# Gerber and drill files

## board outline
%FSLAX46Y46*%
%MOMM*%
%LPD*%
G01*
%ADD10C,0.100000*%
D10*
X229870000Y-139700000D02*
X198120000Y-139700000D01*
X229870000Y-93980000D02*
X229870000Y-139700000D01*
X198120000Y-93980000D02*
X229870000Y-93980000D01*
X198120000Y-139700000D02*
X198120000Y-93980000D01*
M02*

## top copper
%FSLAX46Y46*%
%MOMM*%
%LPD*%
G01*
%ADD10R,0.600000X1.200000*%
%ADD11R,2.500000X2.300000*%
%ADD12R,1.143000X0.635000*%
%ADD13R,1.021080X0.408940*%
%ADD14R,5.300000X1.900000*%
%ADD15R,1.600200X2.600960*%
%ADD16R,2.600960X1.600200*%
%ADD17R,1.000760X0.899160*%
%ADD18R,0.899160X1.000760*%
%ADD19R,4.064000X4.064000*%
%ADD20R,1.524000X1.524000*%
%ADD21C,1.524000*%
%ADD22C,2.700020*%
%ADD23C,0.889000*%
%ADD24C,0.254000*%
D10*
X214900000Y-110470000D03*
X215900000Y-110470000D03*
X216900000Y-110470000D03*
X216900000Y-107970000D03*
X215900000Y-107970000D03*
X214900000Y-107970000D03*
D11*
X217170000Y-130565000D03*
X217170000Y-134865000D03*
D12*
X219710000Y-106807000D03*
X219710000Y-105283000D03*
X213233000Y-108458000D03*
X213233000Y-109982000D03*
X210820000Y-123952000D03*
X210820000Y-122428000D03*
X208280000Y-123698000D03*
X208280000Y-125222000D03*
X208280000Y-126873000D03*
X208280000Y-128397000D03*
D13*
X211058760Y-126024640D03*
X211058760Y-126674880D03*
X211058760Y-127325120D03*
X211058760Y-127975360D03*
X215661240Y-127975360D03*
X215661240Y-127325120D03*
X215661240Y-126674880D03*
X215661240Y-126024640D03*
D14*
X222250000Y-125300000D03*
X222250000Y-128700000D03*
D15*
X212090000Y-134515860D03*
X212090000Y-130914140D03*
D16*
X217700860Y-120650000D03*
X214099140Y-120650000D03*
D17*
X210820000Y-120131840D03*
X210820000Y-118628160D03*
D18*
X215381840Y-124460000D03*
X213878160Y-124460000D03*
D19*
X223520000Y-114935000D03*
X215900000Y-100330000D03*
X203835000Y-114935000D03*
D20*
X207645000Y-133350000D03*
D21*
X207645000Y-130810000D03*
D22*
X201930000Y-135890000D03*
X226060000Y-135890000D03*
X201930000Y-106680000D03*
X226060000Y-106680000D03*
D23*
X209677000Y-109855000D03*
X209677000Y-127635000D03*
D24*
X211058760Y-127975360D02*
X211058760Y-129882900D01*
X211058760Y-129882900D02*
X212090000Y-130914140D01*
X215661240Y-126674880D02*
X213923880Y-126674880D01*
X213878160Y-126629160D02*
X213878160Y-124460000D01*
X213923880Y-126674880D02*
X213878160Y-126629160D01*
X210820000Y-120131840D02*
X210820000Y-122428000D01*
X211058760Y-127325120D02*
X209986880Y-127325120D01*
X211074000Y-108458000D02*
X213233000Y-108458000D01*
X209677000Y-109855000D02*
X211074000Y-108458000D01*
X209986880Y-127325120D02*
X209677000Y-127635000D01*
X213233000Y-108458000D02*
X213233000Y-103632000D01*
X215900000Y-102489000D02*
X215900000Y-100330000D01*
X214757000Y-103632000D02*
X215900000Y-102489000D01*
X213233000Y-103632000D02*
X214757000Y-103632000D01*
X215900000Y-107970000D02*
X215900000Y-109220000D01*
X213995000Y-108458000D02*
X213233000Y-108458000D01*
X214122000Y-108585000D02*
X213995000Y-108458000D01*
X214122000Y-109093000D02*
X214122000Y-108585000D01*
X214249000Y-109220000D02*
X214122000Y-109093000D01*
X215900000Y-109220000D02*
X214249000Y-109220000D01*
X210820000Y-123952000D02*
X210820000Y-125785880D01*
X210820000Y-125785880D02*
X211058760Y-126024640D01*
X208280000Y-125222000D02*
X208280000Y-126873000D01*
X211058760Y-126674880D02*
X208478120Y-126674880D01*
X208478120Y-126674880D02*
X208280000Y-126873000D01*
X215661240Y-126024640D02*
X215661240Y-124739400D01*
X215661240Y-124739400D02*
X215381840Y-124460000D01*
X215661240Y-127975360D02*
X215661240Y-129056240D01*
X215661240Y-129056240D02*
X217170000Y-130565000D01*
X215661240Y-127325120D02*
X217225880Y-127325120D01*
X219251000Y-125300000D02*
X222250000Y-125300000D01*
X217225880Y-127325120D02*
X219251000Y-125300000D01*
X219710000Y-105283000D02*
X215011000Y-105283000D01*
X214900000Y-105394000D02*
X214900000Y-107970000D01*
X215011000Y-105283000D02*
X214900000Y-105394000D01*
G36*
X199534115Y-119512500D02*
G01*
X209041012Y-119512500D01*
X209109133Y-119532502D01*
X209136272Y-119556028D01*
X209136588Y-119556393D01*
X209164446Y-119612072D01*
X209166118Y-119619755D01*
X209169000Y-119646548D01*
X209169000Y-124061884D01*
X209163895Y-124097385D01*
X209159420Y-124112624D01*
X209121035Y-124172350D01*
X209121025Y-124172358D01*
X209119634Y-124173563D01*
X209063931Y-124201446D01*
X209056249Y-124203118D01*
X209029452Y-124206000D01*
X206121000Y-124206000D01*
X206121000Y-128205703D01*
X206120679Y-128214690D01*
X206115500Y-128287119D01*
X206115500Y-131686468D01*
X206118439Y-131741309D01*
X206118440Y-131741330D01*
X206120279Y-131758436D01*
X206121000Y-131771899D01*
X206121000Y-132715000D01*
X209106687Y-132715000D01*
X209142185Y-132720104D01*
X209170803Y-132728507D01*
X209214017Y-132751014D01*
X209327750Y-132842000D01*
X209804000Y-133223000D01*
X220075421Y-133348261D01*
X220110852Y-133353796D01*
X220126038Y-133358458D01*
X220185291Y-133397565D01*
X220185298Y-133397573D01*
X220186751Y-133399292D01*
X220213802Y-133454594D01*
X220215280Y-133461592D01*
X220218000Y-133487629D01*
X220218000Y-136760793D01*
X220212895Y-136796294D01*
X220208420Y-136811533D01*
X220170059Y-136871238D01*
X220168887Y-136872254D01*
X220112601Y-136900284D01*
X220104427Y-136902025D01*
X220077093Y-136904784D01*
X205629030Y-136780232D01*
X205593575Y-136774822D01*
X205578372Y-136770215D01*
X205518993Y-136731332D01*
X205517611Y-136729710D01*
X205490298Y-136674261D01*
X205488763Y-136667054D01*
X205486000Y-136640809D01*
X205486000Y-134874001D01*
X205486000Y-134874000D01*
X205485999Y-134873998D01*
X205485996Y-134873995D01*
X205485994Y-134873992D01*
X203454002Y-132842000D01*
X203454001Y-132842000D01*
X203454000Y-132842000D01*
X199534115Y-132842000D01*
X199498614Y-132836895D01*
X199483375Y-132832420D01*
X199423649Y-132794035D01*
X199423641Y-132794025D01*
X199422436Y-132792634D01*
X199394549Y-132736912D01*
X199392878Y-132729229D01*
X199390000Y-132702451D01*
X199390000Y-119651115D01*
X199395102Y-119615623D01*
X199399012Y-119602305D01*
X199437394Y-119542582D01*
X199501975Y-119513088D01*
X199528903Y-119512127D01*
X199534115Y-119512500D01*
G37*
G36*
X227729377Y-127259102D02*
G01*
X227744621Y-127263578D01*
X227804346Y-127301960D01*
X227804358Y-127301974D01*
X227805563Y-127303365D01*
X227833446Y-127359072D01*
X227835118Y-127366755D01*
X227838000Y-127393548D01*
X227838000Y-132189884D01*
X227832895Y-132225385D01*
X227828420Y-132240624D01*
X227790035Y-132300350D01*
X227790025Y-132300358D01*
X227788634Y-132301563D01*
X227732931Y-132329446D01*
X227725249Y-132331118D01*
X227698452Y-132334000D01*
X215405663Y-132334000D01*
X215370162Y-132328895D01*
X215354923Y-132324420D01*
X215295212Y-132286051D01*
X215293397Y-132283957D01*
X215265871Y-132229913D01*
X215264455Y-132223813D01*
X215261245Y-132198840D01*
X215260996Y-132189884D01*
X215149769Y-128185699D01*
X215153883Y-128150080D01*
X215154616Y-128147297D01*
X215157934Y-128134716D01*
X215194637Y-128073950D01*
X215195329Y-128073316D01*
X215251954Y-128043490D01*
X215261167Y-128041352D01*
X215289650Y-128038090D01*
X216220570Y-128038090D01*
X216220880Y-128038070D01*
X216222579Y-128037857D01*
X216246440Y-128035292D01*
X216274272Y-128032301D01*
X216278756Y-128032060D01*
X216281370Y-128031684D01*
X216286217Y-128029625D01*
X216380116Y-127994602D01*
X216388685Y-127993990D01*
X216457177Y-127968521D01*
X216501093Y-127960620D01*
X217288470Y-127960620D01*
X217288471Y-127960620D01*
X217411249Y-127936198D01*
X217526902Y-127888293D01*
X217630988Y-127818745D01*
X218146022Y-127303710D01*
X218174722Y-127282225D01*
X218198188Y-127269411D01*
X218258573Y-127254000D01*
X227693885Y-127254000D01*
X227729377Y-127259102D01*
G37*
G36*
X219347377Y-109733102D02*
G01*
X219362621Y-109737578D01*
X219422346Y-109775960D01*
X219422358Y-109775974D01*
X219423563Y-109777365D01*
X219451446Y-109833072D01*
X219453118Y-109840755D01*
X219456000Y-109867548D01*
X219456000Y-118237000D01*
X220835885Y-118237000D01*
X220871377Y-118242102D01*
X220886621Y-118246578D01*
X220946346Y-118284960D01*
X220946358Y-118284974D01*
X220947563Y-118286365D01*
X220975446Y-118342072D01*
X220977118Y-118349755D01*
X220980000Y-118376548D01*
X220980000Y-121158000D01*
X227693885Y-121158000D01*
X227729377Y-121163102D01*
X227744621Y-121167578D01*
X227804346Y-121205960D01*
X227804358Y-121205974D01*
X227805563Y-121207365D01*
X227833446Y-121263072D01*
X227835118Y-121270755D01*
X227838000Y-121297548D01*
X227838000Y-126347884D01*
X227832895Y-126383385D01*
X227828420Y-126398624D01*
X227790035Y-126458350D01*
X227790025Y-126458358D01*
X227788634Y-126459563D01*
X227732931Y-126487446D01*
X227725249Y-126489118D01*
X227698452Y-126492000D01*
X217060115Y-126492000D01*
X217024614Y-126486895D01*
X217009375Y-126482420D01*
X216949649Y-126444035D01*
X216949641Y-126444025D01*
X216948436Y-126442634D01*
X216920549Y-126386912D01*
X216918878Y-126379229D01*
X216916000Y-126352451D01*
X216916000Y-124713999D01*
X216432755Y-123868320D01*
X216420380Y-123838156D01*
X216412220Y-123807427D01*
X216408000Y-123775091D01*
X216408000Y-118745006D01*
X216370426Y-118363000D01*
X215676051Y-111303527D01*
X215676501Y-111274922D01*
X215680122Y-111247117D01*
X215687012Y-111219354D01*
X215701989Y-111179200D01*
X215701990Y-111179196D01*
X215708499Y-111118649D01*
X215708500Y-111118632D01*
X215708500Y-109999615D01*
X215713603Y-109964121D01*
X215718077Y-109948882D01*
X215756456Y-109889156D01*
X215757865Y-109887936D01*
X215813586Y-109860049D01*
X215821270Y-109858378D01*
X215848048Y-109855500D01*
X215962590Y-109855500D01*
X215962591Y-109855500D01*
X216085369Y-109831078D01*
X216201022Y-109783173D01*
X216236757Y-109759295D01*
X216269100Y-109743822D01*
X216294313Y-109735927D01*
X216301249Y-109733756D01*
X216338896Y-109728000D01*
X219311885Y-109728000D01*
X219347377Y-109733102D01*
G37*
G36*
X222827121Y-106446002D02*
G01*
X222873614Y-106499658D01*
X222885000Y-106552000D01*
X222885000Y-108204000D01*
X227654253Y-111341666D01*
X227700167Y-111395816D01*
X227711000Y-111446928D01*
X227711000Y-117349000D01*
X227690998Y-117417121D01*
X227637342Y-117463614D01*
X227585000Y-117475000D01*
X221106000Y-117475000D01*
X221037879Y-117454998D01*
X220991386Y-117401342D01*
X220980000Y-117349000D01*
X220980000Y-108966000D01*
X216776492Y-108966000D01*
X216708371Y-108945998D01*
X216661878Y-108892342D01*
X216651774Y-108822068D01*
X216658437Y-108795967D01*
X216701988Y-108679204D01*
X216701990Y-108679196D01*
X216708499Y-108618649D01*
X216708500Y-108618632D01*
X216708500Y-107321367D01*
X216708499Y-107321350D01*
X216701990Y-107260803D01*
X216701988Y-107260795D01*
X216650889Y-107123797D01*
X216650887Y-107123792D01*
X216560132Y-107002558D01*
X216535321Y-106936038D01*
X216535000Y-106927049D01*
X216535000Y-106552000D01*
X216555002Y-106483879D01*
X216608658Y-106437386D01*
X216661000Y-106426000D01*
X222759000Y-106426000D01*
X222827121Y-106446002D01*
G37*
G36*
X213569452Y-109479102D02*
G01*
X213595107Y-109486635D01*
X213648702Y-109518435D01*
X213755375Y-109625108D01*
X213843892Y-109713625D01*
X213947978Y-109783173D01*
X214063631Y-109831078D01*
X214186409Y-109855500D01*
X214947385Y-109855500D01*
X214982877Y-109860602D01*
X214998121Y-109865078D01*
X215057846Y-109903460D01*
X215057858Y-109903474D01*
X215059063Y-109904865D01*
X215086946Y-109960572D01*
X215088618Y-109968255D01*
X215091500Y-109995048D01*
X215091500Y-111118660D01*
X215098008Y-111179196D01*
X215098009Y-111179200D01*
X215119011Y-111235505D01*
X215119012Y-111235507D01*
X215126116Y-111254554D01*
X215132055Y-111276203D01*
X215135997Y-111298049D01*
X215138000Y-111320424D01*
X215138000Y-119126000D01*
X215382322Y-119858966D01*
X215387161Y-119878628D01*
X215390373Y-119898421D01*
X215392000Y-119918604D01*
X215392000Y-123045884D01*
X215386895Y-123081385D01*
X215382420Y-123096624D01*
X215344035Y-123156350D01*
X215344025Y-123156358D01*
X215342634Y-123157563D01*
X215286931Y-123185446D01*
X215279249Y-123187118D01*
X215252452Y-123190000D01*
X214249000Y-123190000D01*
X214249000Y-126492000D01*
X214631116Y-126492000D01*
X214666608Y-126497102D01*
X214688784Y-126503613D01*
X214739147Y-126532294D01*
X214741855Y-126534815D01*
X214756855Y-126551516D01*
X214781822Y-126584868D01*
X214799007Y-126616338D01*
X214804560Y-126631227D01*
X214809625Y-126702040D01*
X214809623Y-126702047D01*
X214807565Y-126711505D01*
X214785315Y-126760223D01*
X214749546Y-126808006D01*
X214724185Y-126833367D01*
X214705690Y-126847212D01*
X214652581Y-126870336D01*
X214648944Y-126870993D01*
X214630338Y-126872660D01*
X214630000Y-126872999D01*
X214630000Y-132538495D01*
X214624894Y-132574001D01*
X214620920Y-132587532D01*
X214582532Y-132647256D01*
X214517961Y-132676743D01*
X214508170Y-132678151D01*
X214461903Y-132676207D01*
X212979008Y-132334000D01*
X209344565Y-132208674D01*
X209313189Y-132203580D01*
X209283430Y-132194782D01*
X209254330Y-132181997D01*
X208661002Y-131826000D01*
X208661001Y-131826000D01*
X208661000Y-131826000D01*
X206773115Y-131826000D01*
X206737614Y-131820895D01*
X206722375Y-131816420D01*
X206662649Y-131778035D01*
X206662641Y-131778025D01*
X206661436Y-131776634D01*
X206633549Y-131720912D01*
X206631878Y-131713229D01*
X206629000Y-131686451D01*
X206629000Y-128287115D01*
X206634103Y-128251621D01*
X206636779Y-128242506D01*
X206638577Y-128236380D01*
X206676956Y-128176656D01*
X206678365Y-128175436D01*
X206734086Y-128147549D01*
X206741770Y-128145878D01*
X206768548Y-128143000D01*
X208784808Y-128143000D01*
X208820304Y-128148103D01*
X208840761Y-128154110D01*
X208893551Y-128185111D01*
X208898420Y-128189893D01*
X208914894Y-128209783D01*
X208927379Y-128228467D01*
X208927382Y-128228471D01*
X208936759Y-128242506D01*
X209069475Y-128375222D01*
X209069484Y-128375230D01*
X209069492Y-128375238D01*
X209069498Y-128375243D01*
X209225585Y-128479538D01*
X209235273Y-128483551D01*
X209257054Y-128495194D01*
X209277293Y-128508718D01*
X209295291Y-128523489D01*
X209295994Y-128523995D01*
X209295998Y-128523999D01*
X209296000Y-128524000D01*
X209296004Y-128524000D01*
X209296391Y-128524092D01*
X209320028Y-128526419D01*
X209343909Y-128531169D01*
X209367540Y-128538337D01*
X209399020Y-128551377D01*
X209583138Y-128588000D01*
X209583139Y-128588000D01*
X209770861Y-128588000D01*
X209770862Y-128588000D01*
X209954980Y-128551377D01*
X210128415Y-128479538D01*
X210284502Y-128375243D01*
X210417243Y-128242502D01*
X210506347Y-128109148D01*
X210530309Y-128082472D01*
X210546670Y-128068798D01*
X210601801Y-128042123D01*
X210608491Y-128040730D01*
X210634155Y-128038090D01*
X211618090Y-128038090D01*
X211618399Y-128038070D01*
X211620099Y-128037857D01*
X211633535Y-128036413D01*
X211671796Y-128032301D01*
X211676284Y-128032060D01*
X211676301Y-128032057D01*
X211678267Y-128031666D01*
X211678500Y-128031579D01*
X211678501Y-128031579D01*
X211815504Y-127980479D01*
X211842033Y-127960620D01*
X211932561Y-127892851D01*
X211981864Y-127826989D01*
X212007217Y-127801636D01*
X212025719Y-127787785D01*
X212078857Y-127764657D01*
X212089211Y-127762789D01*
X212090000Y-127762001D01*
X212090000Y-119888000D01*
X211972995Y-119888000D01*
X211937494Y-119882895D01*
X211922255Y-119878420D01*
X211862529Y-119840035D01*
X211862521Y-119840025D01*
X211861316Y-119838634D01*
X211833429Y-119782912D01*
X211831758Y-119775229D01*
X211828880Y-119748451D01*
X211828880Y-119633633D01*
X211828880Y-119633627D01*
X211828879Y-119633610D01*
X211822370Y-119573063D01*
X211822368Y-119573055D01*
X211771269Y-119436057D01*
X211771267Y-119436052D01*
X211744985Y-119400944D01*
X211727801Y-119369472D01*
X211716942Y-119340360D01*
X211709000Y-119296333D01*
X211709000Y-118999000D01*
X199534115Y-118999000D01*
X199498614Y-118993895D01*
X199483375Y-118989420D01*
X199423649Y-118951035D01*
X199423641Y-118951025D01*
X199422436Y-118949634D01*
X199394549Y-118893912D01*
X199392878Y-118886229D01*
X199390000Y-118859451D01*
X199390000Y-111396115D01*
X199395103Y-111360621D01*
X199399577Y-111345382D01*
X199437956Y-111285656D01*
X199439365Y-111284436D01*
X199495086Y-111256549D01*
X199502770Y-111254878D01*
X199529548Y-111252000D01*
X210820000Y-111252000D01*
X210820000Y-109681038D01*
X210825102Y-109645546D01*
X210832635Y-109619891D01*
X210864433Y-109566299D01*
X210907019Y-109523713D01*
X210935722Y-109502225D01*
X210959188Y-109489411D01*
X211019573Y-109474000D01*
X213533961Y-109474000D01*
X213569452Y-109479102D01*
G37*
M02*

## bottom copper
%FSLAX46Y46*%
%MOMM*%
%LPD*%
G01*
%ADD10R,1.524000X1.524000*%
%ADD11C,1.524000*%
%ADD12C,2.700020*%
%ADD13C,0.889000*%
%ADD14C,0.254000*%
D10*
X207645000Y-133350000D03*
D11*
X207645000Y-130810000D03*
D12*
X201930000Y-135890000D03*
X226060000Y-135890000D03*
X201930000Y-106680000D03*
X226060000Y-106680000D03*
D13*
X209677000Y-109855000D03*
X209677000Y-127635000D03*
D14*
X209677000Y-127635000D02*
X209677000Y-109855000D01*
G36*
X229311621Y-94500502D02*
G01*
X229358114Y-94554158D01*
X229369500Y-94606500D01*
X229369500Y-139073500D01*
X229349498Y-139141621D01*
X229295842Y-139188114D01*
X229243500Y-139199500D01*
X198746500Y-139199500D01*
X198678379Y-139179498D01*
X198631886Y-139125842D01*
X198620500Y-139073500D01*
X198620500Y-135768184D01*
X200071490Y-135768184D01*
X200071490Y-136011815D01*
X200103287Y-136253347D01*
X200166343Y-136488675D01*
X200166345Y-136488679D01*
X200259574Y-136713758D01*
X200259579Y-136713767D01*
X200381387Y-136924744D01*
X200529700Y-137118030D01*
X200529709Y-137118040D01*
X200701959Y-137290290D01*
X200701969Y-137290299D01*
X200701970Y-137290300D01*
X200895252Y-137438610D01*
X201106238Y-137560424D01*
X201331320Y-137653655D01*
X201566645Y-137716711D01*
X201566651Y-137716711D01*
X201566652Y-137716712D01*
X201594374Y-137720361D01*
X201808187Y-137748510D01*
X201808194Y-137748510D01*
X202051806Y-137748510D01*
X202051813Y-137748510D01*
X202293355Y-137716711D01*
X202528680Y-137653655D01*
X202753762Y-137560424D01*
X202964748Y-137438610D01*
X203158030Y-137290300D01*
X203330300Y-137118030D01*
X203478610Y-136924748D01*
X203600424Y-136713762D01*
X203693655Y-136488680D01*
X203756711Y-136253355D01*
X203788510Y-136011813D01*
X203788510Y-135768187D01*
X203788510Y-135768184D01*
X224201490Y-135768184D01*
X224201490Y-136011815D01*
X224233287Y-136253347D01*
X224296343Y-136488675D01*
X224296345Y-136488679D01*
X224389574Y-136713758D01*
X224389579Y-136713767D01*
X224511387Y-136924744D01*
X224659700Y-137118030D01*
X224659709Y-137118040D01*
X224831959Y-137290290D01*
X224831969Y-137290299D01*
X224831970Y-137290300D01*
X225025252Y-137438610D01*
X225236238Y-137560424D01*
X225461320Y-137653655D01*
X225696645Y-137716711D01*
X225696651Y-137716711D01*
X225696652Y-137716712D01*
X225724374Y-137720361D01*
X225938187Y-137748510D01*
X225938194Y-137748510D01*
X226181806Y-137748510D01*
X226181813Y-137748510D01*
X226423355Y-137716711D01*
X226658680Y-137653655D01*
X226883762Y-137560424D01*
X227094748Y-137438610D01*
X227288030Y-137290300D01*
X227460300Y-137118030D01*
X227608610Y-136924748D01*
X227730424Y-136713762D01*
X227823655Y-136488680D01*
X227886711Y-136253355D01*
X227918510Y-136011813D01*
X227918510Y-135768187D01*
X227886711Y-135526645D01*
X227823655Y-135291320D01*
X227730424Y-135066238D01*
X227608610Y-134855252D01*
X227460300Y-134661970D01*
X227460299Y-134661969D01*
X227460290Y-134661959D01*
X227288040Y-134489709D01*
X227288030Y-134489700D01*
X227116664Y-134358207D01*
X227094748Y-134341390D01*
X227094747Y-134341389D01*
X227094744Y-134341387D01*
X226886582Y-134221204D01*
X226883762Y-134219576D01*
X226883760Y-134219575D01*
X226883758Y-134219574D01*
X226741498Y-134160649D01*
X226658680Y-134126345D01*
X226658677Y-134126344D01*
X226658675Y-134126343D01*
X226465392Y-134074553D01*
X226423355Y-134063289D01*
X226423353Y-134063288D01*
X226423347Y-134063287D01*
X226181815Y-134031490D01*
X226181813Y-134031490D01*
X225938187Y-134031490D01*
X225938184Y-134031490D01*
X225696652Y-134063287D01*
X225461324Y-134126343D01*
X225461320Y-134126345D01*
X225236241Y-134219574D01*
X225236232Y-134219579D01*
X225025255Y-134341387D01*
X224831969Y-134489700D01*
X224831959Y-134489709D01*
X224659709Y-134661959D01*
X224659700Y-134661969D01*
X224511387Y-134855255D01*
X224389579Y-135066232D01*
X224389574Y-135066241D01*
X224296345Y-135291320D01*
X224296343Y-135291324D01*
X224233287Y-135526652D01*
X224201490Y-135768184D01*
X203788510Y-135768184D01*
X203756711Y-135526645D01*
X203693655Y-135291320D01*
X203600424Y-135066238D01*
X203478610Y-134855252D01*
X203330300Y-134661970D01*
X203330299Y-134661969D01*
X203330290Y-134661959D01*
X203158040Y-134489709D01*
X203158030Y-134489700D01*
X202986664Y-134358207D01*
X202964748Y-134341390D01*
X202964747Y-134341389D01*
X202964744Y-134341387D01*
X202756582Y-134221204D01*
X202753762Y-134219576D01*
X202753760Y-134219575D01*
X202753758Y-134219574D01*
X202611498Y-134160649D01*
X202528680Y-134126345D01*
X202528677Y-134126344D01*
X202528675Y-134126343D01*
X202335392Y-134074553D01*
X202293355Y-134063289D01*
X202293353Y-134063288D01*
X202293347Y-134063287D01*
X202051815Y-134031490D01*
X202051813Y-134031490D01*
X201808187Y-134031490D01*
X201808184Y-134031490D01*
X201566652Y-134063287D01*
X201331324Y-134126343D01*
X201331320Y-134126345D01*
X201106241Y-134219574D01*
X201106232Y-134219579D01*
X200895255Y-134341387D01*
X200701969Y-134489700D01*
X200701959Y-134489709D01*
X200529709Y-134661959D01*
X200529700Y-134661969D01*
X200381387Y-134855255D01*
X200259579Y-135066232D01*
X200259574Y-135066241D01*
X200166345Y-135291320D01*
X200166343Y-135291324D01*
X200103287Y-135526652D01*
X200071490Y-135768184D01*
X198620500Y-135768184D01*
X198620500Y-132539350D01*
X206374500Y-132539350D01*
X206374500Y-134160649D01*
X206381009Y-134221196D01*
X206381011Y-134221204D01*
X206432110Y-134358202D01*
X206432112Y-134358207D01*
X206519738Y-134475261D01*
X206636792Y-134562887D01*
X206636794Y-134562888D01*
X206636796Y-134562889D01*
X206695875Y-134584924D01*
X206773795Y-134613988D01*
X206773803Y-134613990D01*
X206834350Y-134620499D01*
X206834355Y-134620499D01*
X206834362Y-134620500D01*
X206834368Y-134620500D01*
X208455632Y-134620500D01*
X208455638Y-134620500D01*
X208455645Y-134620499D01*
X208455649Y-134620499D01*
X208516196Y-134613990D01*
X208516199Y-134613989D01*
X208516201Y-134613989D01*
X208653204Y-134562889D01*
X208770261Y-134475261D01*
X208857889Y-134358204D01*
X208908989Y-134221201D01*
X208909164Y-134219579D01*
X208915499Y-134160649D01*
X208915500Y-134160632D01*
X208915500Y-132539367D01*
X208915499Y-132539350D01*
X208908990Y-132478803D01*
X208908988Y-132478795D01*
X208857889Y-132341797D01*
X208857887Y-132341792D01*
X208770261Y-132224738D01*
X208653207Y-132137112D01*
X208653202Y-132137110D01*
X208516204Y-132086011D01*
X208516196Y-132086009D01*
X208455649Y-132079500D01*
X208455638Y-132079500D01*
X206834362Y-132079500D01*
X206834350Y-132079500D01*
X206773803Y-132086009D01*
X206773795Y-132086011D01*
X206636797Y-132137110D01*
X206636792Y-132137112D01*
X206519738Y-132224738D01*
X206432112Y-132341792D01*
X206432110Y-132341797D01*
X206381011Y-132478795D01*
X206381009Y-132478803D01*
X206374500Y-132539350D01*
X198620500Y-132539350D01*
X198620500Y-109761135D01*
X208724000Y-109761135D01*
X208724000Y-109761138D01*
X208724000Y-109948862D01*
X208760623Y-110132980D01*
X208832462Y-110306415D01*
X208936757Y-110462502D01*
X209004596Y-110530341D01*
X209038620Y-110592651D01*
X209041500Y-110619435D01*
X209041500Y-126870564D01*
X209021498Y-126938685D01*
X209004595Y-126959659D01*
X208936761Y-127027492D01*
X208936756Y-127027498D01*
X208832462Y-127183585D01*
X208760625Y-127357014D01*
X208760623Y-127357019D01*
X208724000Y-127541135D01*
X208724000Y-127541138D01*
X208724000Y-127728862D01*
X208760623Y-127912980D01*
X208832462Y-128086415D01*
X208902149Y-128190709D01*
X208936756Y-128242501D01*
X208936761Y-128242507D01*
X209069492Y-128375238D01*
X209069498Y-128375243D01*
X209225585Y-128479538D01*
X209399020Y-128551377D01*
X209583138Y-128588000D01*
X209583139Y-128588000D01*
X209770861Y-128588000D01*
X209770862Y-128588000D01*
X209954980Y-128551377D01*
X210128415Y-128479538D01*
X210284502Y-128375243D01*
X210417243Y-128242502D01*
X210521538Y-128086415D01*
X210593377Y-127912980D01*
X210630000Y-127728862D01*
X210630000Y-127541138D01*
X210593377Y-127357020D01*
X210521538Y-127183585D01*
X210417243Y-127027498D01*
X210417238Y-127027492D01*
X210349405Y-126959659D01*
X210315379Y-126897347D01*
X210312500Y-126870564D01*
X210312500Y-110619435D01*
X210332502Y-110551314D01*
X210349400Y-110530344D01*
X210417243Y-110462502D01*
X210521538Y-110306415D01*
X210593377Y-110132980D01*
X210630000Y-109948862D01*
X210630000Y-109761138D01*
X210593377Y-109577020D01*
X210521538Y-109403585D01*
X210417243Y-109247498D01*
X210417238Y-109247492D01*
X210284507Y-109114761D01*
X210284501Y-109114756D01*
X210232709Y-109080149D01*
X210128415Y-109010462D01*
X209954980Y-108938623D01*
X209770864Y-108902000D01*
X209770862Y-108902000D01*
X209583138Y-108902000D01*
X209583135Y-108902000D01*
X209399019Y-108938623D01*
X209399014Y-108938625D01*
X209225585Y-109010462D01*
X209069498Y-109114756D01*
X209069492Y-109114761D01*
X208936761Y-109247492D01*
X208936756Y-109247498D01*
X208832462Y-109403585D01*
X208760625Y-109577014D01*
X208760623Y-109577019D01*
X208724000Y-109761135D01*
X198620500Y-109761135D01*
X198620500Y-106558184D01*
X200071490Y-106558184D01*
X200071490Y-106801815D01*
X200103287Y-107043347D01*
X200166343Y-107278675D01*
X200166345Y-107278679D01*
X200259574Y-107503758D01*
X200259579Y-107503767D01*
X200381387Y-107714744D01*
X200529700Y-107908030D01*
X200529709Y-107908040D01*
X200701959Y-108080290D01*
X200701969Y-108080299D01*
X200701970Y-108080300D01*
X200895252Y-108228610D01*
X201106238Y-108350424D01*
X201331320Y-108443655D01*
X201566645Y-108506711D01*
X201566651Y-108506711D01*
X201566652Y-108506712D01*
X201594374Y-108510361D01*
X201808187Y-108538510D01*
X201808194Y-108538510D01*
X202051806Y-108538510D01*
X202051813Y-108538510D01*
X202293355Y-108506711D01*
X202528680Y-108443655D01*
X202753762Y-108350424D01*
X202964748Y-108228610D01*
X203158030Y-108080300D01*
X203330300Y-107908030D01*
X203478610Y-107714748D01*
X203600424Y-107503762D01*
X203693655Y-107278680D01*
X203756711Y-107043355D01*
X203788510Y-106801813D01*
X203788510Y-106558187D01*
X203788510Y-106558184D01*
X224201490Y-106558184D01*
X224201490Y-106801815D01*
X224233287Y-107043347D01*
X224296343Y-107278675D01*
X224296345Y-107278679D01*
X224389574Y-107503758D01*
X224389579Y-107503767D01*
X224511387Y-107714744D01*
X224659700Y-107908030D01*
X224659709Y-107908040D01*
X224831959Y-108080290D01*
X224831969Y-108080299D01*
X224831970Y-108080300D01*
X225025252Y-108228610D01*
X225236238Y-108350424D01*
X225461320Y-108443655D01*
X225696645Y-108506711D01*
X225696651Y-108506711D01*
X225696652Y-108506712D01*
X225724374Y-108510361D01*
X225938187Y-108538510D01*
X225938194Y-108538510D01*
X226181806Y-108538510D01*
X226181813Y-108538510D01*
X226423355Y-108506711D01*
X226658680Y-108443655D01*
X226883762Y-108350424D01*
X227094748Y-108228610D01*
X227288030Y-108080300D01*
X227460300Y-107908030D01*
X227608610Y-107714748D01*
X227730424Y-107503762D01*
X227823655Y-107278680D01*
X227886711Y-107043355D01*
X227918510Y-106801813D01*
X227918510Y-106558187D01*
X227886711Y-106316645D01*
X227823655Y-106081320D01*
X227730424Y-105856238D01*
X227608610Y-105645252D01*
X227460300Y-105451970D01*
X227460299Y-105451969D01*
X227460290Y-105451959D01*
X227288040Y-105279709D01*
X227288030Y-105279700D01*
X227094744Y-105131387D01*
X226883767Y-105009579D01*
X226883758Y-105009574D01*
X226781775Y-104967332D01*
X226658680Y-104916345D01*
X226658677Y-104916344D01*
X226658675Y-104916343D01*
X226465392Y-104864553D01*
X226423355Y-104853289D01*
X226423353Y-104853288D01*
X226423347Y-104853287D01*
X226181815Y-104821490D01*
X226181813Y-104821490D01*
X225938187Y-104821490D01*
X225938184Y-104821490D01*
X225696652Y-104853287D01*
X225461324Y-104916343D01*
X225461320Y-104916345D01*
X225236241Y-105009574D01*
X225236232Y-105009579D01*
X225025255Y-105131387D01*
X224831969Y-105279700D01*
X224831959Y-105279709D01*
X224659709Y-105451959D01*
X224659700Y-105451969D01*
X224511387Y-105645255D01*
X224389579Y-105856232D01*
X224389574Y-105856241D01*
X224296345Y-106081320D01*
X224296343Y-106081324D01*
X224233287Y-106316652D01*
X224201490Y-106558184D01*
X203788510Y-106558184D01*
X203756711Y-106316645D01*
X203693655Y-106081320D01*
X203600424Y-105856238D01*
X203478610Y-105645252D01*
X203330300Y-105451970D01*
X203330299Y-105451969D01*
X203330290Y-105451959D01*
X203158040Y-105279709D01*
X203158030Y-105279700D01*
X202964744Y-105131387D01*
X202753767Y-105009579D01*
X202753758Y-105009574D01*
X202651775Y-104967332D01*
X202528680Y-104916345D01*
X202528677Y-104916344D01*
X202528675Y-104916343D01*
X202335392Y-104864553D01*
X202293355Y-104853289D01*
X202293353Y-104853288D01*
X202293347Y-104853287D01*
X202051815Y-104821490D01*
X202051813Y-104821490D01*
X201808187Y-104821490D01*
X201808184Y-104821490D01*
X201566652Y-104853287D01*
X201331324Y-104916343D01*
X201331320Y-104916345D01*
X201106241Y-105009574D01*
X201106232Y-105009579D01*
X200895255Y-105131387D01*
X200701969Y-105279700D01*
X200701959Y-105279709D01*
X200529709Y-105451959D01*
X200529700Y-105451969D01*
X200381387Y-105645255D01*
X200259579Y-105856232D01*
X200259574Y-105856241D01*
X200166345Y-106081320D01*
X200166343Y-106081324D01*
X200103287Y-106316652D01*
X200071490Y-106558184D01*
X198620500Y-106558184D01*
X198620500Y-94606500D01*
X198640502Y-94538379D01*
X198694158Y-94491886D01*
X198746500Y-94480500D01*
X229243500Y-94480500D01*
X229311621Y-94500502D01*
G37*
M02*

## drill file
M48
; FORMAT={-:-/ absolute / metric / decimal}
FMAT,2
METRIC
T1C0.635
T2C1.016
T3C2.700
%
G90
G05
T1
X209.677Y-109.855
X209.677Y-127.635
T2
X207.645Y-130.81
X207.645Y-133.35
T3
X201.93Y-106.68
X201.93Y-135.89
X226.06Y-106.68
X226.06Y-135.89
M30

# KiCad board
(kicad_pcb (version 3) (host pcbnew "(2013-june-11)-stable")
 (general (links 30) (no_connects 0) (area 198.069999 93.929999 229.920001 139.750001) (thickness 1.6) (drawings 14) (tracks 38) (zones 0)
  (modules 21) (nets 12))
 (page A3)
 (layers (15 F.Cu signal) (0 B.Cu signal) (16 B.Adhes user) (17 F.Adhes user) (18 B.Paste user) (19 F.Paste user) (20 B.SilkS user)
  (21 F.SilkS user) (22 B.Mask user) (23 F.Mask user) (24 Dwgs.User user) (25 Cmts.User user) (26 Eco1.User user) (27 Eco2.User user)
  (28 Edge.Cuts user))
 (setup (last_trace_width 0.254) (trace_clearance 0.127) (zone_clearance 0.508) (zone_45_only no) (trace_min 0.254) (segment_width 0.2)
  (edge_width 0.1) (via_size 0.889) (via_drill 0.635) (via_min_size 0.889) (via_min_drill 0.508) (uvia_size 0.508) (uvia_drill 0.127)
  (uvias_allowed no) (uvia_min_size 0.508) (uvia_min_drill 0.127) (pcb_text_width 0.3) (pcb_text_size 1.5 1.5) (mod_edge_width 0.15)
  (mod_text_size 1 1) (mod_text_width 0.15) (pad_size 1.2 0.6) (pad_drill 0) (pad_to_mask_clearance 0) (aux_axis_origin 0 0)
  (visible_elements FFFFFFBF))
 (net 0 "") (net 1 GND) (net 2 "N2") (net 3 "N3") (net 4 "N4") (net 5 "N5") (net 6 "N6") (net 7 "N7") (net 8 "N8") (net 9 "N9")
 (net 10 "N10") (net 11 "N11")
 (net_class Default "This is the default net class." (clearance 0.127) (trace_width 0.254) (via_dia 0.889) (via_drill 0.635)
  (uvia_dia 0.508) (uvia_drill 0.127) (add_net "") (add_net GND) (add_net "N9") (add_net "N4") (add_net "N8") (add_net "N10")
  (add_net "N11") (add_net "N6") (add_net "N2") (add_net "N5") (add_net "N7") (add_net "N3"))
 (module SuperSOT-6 (layer F.Cu) (at 215.9 109.22 90)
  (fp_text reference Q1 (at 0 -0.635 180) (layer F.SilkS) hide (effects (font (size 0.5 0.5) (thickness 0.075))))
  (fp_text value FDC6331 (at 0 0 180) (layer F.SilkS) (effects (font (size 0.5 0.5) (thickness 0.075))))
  (pad 1 smd rect (at -1.25 -1 90) (size 1.2 0.6) (layers F.Cu F.Paste F.Mask) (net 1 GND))
  (pad 2 smd rect (at -1.25 0 90) (size 1.2 0.6) (layers F.Cu F.Paste F.Mask) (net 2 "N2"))
  (pad 3 smd rect (at -1.25 1 90) (size 1.2 0.6) (layers F.Cu F.Paste F.Mask) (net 2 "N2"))
  (pad 4 smd rect (at 1.25 1 90) (size 1.2 0.6) (layers F.Cu F.Paste F.Mask) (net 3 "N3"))
  (pad 5 smd rect (at 1.25 0 90) (size 1.2 0.6) (layers F.Cu F.Paste F.Mask) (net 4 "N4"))
  (pad 6 smd rect (at 1.25 -1 90) (size 1.2 0.6) (layers F.Cu F.Paste F.Mask) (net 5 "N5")))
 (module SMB (layer F.Cu) (at 217.17 132.715 90)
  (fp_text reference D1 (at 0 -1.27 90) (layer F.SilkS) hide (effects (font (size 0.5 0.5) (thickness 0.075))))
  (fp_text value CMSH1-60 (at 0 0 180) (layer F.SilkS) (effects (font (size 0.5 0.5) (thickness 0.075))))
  (pad 1 smd rect (at 2.15 0 90) (size 2.3 2.5) (layers F.Cu F.Paste F.Mask) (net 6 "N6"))
  (pad 2 smd rect (at -2.15 0 90) (size 2.3 2.5) (layers F.Cu F.Paste F.Mask) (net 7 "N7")))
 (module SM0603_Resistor (layer F.Cu) (at 219.71 106.045 90)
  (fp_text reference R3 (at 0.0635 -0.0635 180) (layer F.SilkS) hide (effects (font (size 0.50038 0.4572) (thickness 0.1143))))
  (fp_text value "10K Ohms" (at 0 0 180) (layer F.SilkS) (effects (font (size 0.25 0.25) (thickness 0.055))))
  (pad 1 smd rect (at -0.762 0 90) (size 0.635 1.143) (layers F.Cu F.Paste F.Mask) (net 3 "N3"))
  (pad 2 smd rect (at 0.762 0 90) (size 0.635 1.143) (layers F.Cu F.Paste F.Mask) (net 5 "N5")))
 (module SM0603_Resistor (layer F.Cu) (at 213.233 109.22 270)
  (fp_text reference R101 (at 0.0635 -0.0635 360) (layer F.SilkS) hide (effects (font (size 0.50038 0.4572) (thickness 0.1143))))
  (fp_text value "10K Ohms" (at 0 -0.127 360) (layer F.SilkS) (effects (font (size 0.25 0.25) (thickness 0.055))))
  (pad 1 smd rect (at -0.762 0 270) (size 0.635 1.143) (layers F.Cu F.Paste F.Mask) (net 4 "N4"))
  (pad 2 smd rect (at 0.762 0 270) (size 0.635 1.143) (layers F.Cu F.Paste F.Mask) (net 1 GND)))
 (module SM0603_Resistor (layer F.Cu) (at 210.82 123.19 90)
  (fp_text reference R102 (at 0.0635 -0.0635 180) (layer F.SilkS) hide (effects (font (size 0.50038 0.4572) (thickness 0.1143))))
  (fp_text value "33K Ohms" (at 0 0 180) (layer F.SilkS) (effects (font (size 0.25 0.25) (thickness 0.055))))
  (pad 1 smd rect (at -0.762 0 90) (size 0.635 1.143) (layers F.Cu F.Paste F.Mask) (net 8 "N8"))
  (pad 2 smd rect (at 0.762 0 90) (size 0.635 1.143) (layers F.Cu F.Paste F.Mask) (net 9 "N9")))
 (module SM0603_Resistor (layer F.Cu) (at 208.28 124.46 270)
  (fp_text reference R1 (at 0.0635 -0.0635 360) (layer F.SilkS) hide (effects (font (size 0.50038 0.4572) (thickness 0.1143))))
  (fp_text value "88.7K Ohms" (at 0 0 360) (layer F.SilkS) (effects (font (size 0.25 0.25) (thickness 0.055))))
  (pad 1 smd rect (at -0.762 0 270) (size 0.635 1.143) (layers F.Cu F.Paste F.Mask) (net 7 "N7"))
  (pad 2 smd rect (at 0.762 0 270) (size 0.635 1.143) (layers F.Cu F.Paste F.Mask) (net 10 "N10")))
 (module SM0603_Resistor (layer F.Cu) (at 208.28 127.635 270)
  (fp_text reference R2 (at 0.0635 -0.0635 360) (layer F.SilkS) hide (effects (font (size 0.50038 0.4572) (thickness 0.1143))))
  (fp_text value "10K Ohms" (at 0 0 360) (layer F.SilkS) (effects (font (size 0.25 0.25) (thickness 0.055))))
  (pad 1 smd rect (at -0.762 0 270) (size 0.635 1.143) (layers F.Cu F.Paste F.Mask) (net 10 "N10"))
  (pad 2 smd rect (at 0.762 0 270) (size 0.635 1.143) (layers F.Cu F.Paste F.Mask) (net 1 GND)))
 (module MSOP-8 (layer F.Cu) (at 213.36 127 270)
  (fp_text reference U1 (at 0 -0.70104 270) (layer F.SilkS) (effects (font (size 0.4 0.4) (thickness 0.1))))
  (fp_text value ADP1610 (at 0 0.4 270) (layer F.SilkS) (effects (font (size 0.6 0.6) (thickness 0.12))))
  (pad 1 smd rect (at -0.97536 2.30124 270) (size 0.40894 1.02108) (layers F.Cu F.Paste F.Mask) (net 8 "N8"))
  (pad 2 smd rect (at -0.32512 2.30124 270) (size 0.40894 1.02108) (layers F.Cu F.Paste F.Mask) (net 10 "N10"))
  (pad 3 smd rect (at 0.32512 2.30124 270) (size 0.40894 1.02108) (layers F.Cu F.Paste F.Mask) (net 4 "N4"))
  (pad 4 smd rect (at 0.97536 2.30124 270) (size 0.40894 1.02108) (layers F.Cu F.Paste F.Mask) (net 1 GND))
  (pad 5 smd rect (at 0.97536 -2.30124 270) (size 0.40894 1.02108) (layers F.Cu F.Paste F.Mask) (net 6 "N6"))
  (pad 6 smd rect (at 0.32512 -2.30124 270) (size 0.40894 1.02108) (layers F.Cu F.Paste F.Mask) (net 2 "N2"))
  (pad 7 smd rect (at -0.32512 -2.30124 270) (size 0.40894 1.02108) (layers F.Cu F.Paste F.Mask) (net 1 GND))
  (pad 8 smd rect (at -0.97536 -2.30124 270) (size 0.40894 1.02108) (layers F.Cu F.Paste F.Mask) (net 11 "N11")))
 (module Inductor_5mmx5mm (layer F.Cu) (at 222.25 127)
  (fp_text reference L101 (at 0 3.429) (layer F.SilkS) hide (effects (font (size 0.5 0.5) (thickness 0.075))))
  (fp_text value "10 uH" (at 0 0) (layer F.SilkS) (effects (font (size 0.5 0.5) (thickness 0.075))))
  (pad 1 smd rect (at 0 -1.7) (size 5.3 1.9) (layers F.Cu F.Paste F.Mask) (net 2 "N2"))
  (pad 2 smd rect (at 0 1.7) (size 5.3 1.9) (layers F.Cu F.Paste F.Mask) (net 6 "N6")))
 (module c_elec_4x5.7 (layer F.Cu) (at 212.09 132.715 270)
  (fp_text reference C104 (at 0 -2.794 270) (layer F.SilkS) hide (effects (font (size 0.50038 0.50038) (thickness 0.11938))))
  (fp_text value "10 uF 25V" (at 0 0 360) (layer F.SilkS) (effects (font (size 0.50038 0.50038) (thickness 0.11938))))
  (pad 1 smd rect (at 1.80086 0 270) (size 2.60096 1.6002) (layers F.Cu F.Paste F.Mask) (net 7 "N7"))
  (pad 2 smd rect (at -1.80086 0 270) (size 2.60096 1.6002) (layers F.Cu F.Paste F.Mask) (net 1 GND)))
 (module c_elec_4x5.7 (layer F.Cu) (at 215.9 120.65)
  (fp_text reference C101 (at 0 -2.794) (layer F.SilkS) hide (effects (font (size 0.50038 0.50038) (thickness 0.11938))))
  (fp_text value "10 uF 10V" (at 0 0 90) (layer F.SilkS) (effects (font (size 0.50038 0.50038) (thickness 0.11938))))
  (pad 1 smd rect (at 1.80086 0) (size 2.60096 1.6002) (layers F.Cu F.Paste F.Mask) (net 2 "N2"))
  (pad 2 smd rect (at -1.80086 0) (size 2.60096 1.6002) (layers F.Cu F.Paste F.Mask) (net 1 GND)))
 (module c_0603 (layer F.Cu) (at 210.82 119.38 270)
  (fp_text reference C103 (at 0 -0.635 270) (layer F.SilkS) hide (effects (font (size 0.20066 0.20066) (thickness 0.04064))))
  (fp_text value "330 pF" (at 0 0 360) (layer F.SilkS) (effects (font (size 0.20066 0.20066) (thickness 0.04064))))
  (pad 1 smd rect (at 0.75184 0 270) (size 0.89916 1.00076) (layers F.Cu F.Paste F.Mask) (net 9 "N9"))
  (pad 2 smd rect (at -0.75184 0 270) (size 0.89916 1.00076) (layers F.Cu F.Paste F.Mask) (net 1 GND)))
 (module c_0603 (layer F.Cu) (at 214.63 124.46)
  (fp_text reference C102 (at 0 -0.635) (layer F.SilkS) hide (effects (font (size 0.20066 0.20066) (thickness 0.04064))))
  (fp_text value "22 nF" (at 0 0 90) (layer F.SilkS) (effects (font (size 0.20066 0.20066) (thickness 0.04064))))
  (pad 1 smd rect (at 0.75184 0) (size 0.89916 1.00076) (layers F.Cu F.Paste F.Mask) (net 11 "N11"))
  (pad 2 smd rect (at -0.75184 0) (size 0.89916 1.00076) (layers F.Cu F.Paste F.Mask) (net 1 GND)))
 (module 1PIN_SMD (layer F.Cu) (at 223.52 114.935 270)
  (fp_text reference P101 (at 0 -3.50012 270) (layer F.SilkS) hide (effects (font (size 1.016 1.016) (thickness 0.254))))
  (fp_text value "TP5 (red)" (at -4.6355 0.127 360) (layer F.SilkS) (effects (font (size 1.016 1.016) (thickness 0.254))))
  (pad 1 smd rect (at 0 0 270) (size 4.064 4.064) (layers F.Cu F.Paste F.SilkS F.Mask) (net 3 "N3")))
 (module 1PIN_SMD (layer F.Cu) (at 215.9 100.33 270)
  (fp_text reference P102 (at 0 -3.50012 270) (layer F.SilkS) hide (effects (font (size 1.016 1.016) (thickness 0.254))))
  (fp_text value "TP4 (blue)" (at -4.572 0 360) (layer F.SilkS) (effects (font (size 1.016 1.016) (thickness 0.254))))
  (pad 1 smd rect (at 0 0 270) (size 4.064 4.064) (layers F.Cu F.Paste F.SilkS F.Mask) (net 4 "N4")))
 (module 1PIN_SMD (layer F.Cu) (at 203.835 114.935 90)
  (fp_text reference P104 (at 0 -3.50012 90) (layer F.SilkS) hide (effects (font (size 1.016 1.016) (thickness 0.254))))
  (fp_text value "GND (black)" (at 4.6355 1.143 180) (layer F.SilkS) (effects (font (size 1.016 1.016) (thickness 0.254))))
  (pad 1 smd rect (at 0 0 90) (size 4.064 4.064) (layers F.Cu F.Paste F.SilkS F.Mask) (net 1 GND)))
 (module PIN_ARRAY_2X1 (layer F.Cu) (at 207.645 132.08 90)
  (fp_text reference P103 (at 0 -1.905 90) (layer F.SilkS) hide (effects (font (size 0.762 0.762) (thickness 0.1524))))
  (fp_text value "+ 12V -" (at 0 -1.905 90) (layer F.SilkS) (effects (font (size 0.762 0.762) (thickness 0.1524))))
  (pad 1 thru_hole rect (at -1.27 0 90) (size 1.524 1.524) (drill 1.016) (layers *.Cu *.Mask F.SilkS) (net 7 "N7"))
  (pad 2 thru_hole circle (at 1.27 0 90) (size 1.524 1.524) (drill 1.016) (layers *.Cu *.Mask F.SilkS) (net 1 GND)))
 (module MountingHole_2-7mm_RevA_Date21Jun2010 (layer F.Cu) (at 201.93 135.89)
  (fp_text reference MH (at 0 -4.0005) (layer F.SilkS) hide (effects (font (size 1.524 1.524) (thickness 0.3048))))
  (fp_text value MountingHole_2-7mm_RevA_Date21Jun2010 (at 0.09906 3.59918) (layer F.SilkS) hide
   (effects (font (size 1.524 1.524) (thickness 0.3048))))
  (pad 1 thru_hole circle (at 0 0) (size 2.70002 2.70002) (drill 2.70002) (layers)))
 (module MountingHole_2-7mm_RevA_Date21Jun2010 (layer F.Cu) (at 226.06 135.89)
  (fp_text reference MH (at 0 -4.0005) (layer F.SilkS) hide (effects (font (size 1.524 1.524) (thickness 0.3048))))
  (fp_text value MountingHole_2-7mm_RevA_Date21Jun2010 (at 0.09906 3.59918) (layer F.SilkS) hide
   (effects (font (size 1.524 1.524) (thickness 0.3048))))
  (pad 1 thru_hole circle (at 0 0) (size 2.70002 2.70002) (drill 2.70002) (layers)))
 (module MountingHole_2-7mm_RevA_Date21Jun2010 (layer F.Cu) (at 201.93 106.68)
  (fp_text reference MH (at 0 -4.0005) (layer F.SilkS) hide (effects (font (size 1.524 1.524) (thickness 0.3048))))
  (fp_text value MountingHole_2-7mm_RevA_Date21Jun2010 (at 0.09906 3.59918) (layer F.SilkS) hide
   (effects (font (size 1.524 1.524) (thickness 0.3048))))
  (pad 1 thru_hole circle (at 0 0) (size 2.70002 2.70002) (drill 2.70002) (layers)))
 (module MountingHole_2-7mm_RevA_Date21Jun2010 (layer F.Cu) (at 226.06 106.68)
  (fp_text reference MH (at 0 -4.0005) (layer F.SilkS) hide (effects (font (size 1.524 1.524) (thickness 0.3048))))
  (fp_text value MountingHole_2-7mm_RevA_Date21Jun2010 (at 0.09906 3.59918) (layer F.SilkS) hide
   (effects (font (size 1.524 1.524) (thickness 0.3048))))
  (pad 1 thru_hole circle (at 0 0) (size 2.70002 2.70002) (drill 2.70002) (layers)))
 (gr_line (start 229.87 139.7) (end 198.12 139.7) (angle 90) (layer Edge.Cuts) (width 0.1))
 (gr_line (start 229.87 93.98) (end 229.87 139.7) (angle 90) (layer Edge.Cuts) (width 0.1))
 (gr_line (start 198.12 93.98) (end 229.87 93.98) (angle 90) (layer Edge.Cuts) (width 0.1))
 (gr_line (start 198.12 139.7) (end 198.12 93.98) (angle 90) (layer Edge.Cuts) (width 0.1))
 (segment (start 211.05876 127.97536) (end 211.05876 129.8829) (width 0.254) (layer F.Cu) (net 1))
 (segment (start 211.05876 129.8829) (end 212.09 130.91414) (width 0.254) (layer F.Cu) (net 1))
 (segment (start 215.66124 126.67488) (end 213.92388 126.67488) (width 0.254) (layer F.Cu) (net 1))
 (segment (start 213.87816 126.62916) (end 213.87816 124.46) (width 0.254) (layer F.Cu) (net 1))
 (segment (start 213.92388 126.67488) (end 213.87816 126.62916) (width 0.254) (layer F.Cu) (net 1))
 (segment (start 210.82 120.13184) (end 210.82 122.428) (width 0.254) (layer F.Cu) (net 9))
 (segment (start 211.05876 127.32512) (end 209.98688 127.32512) (width 0.254) (layer F.Cu) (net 4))
 (segment (start 211.074 108.458) (end 213.233 108.458) (width 0.254) (layer F.Cu) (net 4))
 (segment (start 209.677 109.855) (end 211.074 108.458) (width 0.254) (layer F.Cu) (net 4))
 (via (at 209.677 109.855) (size 0.889) (layers F.Cu B.Cu) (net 4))
 (segment (start 209.677 127.635) (end 209.677 109.855) (width 0.254) (layer B.Cu) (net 4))
 (via (at 209.677 127.635) (size 0.889) (layers F.Cu B.Cu) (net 4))
 (segment (start 209.98688 127.32512) (end 209.677 127.635) (width 0.254) (layer F.Cu) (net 4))
 (segment (start 213.233 108.458) (end 213.233 103.632) (width 0.254) (layer F.Cu) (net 4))
 (segment (start 215.9 102.489) (end 215.9 100.33) (width 0.254) (layer F.Cu) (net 4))
 (segment (start 214.757 103.632) (end 215.9 102.489) (width 0.254) (layer F.Cu) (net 4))
 (segment (start 213.233 103.632) (end 214.757 103.632) (width 0.254) (layer F.Cu) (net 4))
 (segment (start 215.9 107.97) (end 215.9 109.22) (width 0.254) (layer F.Cu) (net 4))
 (segment (start 213.995 108.458) (end 213.233 108.458) (width 0.254) (layer F.Cu) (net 4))
 (segment (start 214.122 108.585) (end 213.995 108.458) (width 0.254) (layer F.Cu) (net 4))
 (segment (start 214.122 109.093) (end 214.122 108.585) (width 0.254) (layer F.Cu) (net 4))
 (segment (start 214.249 109.22) (end 214.122 109.093) (width 0.254) (layer F.Cu) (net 4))
 (segment (start 215.9 109.22) (end 214.249 109.22) (width 0.254) (layer F.Cu) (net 4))
 (segment (start 210.82 123.952) (end 210.82 125.78588) (width 0.254) (layer F.Cu) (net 8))
 (segment (start 210.82 125.78588) (end 211.05876 126.02464) (width 0.254) (layer F.Cu) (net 8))
 (segment (start 208.28 125.222) (end 208.28 126.873) (width 0.254) (layer F.Cu) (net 10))
 (segment (start 211.05876 126.67488) (end 208.47812 126.67488) (width 0.254) (layer F.Cu) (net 10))
 (segment (start 208.47812 126.67488) (end 208.28 126.873) (width 0.254) (layer F.Cu) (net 10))
 (segment (start 215.66124 126.02464) (end 215.66124 124.7394) (width 0.254) (layer F.Cu) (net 11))
 (segment (start 215.66124 124.7394) (end 215.38184 124.46) (width 0.254) (layer F.Cu) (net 11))
 (segment (start 215.66124 127.97536) (end 215.66124 129.05624) (width 0.254) (layer F.Cu) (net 6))
 (segment (start 215.66124 129.05624) (end 217.17 130.565) (width 0.254) (layer F.Cu) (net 6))
 (segment (start 215.66124 127.32512) (end 217.22588 127.32512) (width 0.254) (layer F.Cu) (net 2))
 (segment (start 219.251 125.3) (end 222.25 125.3) (width 0.254) (layer F.Cu) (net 2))
 (segment (start 217.22588 127.32512) (end 219.251 125.3) (width 0.254) (layer F.Cu) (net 2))
 (segment (start 219.71 105.283) (end 215.011 105.283) (width 0.254) (layer F.Cu) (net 5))
 (segment (start 214.9 105.394) (end 214.9 107.97) (width 0.254) (layer F.Cu) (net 5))
 (segment (start 215.011 105.283) (end 214.9 105.394) (width 0.254) (layer F.Cu) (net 5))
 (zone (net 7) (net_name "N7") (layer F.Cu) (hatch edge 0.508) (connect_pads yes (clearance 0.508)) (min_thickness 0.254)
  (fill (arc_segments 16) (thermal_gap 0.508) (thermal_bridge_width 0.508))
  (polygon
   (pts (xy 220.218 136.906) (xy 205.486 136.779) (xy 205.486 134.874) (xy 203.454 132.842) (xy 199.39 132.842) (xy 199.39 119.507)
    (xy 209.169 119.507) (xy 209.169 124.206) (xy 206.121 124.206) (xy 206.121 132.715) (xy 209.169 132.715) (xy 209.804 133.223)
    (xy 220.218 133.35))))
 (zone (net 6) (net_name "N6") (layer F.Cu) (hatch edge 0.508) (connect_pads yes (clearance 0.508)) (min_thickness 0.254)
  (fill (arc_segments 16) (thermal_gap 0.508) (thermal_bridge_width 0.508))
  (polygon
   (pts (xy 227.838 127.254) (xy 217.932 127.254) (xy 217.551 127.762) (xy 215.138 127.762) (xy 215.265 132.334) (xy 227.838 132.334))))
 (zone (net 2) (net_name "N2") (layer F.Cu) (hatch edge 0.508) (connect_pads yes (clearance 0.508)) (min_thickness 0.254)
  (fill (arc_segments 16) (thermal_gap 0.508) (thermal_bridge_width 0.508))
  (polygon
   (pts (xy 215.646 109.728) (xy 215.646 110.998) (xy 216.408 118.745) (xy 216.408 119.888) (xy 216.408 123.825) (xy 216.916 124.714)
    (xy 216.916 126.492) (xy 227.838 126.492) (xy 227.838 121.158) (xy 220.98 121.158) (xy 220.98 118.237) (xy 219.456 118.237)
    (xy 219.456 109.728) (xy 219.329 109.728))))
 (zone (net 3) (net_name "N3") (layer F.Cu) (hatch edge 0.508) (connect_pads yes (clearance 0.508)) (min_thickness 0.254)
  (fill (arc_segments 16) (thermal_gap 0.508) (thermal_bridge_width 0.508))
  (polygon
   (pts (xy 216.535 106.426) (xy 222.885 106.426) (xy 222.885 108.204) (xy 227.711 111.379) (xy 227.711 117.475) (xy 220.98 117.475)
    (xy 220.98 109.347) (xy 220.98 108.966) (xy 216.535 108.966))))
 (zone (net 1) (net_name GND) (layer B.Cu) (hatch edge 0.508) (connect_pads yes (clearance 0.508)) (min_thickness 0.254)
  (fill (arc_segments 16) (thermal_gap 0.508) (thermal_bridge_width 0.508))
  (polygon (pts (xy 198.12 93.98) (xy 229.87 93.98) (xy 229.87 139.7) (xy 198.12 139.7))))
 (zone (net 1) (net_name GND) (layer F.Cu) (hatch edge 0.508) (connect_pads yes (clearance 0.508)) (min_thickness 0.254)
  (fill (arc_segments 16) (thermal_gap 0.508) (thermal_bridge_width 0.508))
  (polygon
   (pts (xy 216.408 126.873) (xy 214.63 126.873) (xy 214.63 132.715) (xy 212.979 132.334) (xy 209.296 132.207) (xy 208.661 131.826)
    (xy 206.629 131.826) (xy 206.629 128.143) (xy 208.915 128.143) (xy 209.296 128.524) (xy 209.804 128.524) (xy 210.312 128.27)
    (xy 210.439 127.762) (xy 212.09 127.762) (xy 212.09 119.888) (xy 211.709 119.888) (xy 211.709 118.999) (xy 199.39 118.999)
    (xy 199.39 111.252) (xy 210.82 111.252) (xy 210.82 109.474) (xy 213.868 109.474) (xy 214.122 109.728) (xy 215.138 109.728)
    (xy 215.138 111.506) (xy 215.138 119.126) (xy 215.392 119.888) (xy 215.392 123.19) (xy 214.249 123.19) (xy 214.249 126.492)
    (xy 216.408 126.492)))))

